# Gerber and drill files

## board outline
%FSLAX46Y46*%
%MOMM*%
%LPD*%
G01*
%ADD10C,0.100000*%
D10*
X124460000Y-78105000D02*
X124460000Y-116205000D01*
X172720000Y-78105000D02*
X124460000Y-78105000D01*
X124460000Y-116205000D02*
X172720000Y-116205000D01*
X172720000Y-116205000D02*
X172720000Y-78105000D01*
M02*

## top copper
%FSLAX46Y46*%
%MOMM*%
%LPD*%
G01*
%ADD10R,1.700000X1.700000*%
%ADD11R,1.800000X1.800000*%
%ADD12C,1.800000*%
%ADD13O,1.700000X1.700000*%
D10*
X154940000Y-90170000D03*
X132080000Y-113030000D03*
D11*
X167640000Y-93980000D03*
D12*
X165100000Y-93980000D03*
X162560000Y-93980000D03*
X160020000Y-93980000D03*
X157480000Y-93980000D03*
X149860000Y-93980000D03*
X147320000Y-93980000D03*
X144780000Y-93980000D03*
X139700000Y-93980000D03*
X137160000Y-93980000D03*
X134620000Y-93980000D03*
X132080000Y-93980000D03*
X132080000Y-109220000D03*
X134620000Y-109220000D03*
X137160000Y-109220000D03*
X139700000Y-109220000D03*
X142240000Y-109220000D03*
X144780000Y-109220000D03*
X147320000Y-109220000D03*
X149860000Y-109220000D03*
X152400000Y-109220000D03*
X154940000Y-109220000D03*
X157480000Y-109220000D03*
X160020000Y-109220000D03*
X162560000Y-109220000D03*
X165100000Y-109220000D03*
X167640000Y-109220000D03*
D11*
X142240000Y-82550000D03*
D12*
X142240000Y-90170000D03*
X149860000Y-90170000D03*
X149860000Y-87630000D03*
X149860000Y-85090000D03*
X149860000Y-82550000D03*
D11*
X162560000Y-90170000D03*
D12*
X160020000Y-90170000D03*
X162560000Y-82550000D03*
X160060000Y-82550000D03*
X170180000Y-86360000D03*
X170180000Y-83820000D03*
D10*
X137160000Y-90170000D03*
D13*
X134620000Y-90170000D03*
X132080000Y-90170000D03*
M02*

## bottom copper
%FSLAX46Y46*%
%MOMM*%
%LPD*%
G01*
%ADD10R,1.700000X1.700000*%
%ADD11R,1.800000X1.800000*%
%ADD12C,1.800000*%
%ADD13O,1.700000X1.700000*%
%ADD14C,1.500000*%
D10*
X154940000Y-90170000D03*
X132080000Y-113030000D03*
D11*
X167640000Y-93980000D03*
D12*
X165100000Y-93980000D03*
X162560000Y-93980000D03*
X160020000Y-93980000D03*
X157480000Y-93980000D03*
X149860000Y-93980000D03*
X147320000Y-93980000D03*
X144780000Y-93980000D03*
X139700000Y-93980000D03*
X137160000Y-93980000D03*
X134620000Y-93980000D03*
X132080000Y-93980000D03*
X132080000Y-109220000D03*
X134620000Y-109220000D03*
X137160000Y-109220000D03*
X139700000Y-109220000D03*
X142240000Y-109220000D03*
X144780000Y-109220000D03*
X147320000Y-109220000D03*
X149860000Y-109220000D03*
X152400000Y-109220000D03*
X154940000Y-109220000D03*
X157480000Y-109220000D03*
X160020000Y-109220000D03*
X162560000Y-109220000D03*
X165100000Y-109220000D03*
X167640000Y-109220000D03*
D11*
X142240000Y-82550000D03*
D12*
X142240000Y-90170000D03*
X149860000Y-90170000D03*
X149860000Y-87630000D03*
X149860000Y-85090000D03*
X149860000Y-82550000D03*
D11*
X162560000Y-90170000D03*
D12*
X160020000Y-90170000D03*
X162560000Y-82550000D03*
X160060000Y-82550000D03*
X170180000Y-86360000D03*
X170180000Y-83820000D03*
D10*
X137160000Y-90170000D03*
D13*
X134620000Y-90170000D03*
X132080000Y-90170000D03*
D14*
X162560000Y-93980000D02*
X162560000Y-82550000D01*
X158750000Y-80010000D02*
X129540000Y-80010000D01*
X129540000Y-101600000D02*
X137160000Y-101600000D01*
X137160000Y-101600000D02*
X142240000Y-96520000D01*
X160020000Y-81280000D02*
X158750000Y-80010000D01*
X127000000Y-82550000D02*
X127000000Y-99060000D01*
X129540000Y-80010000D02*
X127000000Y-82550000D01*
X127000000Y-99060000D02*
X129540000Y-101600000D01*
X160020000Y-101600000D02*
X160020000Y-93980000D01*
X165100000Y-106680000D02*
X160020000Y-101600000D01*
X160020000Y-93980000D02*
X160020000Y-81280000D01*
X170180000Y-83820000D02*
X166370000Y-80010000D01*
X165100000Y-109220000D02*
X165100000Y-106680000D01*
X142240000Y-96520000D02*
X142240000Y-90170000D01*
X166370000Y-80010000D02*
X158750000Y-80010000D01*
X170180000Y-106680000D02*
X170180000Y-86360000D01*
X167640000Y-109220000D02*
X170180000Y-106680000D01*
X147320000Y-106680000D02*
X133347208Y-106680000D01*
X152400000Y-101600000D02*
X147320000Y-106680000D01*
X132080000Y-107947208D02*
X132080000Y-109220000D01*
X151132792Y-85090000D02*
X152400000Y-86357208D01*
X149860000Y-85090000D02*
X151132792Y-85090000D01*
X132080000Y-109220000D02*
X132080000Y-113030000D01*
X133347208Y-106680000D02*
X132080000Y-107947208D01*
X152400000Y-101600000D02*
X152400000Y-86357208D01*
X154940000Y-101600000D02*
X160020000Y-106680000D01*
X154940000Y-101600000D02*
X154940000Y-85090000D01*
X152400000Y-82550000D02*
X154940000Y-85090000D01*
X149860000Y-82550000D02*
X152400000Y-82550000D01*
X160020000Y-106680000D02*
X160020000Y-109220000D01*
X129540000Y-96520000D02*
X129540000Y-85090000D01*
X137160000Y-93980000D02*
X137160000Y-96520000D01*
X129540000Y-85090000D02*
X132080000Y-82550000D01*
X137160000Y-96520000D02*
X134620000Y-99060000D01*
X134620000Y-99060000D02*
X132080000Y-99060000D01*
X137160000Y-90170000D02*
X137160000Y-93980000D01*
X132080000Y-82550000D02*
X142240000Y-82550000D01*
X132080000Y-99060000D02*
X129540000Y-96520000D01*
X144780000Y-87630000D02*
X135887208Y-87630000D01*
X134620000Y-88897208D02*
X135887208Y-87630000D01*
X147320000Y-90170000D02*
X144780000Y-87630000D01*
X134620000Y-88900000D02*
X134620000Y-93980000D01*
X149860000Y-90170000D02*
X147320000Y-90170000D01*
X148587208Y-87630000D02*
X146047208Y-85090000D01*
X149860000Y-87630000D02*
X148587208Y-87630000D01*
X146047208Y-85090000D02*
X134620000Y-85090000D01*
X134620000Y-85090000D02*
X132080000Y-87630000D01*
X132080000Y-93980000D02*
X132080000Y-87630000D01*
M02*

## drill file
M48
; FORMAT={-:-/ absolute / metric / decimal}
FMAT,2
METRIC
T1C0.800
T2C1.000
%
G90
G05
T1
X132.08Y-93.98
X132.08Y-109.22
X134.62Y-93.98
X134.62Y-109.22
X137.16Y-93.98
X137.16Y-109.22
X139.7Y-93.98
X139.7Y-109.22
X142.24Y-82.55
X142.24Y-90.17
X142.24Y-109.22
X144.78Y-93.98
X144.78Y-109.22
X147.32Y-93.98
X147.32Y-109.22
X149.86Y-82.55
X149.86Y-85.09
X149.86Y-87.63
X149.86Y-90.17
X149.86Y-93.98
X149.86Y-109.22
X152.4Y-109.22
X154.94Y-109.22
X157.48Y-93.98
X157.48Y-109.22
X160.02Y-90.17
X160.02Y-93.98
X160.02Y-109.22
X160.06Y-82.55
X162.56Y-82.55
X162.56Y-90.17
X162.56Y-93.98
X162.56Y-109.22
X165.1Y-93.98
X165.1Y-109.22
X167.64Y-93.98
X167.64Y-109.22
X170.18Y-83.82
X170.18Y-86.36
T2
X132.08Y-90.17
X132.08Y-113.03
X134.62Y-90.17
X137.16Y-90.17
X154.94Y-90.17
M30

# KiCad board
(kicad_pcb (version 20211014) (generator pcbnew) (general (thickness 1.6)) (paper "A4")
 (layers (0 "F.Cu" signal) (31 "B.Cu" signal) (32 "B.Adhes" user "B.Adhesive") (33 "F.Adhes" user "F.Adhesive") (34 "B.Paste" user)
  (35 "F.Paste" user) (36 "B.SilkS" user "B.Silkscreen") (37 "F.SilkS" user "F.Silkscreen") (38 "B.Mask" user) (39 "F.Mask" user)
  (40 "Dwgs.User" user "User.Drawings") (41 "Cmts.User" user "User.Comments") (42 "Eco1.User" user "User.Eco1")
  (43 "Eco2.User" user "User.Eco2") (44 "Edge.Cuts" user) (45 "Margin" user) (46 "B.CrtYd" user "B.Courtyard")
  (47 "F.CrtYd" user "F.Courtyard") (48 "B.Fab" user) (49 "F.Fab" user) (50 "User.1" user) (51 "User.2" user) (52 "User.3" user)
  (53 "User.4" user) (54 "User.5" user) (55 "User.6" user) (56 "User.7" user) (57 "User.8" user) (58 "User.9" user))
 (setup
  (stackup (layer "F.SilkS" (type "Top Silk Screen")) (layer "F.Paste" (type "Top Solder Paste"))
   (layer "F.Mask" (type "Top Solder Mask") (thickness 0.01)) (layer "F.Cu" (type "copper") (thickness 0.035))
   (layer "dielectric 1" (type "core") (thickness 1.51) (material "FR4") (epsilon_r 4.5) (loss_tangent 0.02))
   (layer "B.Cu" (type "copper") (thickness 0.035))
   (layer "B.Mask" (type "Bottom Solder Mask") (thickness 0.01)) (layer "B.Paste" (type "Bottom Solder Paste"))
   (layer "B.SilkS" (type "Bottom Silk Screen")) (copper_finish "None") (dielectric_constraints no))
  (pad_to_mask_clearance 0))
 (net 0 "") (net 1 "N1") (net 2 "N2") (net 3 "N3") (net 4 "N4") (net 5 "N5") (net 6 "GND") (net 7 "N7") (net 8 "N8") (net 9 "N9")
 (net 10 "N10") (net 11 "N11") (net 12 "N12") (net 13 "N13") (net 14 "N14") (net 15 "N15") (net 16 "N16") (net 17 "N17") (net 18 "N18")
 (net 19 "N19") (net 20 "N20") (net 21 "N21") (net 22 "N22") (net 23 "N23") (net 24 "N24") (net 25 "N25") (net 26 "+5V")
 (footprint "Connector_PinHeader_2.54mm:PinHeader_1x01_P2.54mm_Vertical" (layer "F.Cu") (at 154.94 90.17)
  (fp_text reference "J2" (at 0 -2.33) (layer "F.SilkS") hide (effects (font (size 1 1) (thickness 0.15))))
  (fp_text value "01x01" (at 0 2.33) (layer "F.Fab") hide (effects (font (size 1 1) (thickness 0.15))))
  (pad "1" thru_hole rect (at 0 0) (size 1.7 1.7) (drill 1) (layers *.Cu *.Mask) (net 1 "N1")))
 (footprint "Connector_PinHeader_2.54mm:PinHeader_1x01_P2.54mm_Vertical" (layer "F.Cu") (at 132.08 113.03 -90)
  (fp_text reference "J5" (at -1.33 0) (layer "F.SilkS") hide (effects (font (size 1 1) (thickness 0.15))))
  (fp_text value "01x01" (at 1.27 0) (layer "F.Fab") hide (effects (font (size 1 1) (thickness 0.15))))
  (pad "1" thru_hole rect (at 0 0 270) (size 1.7 1.7) (drill 1) (layers *.Cu *.Mask) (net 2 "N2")))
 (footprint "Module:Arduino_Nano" (layer "F.Cu") (at 167.64 93.98 -90)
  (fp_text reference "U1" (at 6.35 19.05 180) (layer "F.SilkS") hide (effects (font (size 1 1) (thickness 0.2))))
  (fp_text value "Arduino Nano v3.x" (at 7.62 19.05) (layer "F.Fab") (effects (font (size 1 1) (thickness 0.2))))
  (pad "1" thru_hole rect (at 0 0 270) (size 1.8 1.8) (drill 0.8) (layers *.Cu *.Mask) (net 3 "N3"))
  (pad "2" thru_hole circle (at 0 2.54 270) (size 1.8 1.8) (drill 0.8) (layers *.Cu *.Mask) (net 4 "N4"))
  (pad "3" thru_hole circle (at 0 5.08 270) (size 1.8 1.8) (drill 0.8) (layers *.Cu *.Mask) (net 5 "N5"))
  (pad "4" thru_hole circle (at 0 7.62 270) (size 1.8 1.8) (drill 0.8) (layers *.Cu *.Mask) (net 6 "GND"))
  (pad "5" thru_hole circle (at 0 10.16 270) (size 1.8 1.8) (drill 0.8) (layers *.Cu *.Mask) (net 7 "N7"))
  (pad "8" thru_hole circle (at 0 17.78 270) (size 1.8 1.8) (drill 0.8) (layers *.Cu *.Mask) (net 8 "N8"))
  (pad "9" thru_hole circle (at 0 20.32 270) (size 1.8 1.8) (drill 0.8) (layers *.Cu *.Mask) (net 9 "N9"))
  (pad "10" thru_hole circle (at 0 22.86 270) (size 1.8 1.8) (drill 0.8) (layers *.Cu *.Mask) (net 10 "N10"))
  (pad "12" thru_hole circle (at 0 27.94 270) (size 1.8 1.8) (drill 0.8) (layers *.Cu *.Mask) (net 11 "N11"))
  (pad "13" thru_hole circle (at 0 30.48 270) (size 1.8 1.8) (drill 0.8) (layers *.Cu *.Mask) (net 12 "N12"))
  (pad "14" thru_hole circle (at 0 33.02 270) (size 1.8 1.8) (drill 0.8) (layers *.Cu *.Mask) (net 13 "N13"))
  (pad "15" thru_hole circle (at 0 35.56 270) (size 1.8 1.8) (drill 0.8) (layers *.Cu *.Mask) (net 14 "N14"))
  (pad "16" thru_hole circle (at 15.24 35.56 270) (size 1.8 1.8) (drill 0.8) (layers *.Cu *.Mask) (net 2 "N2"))
  (pad "17" thru_hole circle (at 15.24 33.02 270) (size 1.8 1.8) (drill 0.8) (layers *.Cu *.Mask) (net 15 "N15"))
  (pad "18" thru_hole circle (at 15.24 30.48 270) (size 1.8 1.8) (drill 0.8) (layers *.Cu *.Mask) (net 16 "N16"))
  (pad "19" thru_hole circle (at 15.24 27.94 270) (size 1.8 1.8) (drill 0.8) (layers *.Cu *.Mask) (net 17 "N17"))
  (pad "20" thru_hole circle (at 15.24 25.4 270) (size 1.8 1.8) (drill 0.8) (layers *.Cu *.Mask) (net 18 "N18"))
  (pad "21" thru_hole circle (at 15.24 22.86 270) (size 1.8 1.8) (drill 0.8) (layers *.Cu *.Mask) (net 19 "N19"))
  (pad "22" thru_hole circle (at 15.24 20.32 270) (size 1.8 1.8) (drill 0.8) (layers *.Cu *.Mask) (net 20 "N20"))
  (pad "23" thru_hole circle (at 15.24 17.78 270) (size 1.8 1.8) (drill 0.8) (layers *.Cu *.Mask) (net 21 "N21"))
  (pad "24" thru_hole circle (at 15.24 15.24 270) (size 1.8 1.8) (drill 0.8) (layers *.Cu *.Mask) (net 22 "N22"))
  (pad "25" thru_hole circle (at 15.24 12.7 270) (size 1.8 1.8) (drill 0.8) (layers *.Cu *.Mask) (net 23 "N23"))
  (pad "26" thru_hole circle (at 15.24 10.16 270) (size 1.8 1.8) (drill 0.8) (layers *.Cu *.Mask) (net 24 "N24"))
  (pad "27" thru_hole circle (at 15.24 7.62 270) (size 1.8 1.8) (drill 0.8) (layers *.Cu *.Mask) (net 1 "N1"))
  (pad "28" thru_hole circle (at 15.24 5.08 270) (size 1.8 1.8) (drill 0.8) (layers *.Cu *.Mask) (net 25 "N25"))
  (pad "29" thru_hole circle (at 15.24 2.54 270) (size 1.8 1.8) (drill 0.8) (layers *.Cu *.Mask) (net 6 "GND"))
  (pad "30" thru_hole circle (at 15.24 0 270) (size 1.8 1.8) (drill 0.8) (layers *.Cu *.Mask) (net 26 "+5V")))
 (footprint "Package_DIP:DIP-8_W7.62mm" (layer "F.Cu") (at 142.24 82.55)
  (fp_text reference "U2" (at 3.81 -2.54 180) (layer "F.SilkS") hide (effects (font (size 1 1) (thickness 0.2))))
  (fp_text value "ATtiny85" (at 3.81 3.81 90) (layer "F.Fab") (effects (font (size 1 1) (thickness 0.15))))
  (pad "1" thru_hole rect (at 0 0) (size 1.8 1.8) (drill 0.8) (layers *.Cu *.Mask) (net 12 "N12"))
  (pad "4" thru_hole circle (at 0 7.62) (size 1.8 1.8) (drill 0.8) (layers *.Cu *.Mask) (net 6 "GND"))
  (pad "5" thru_hole circle (at 7.62 7.62) (size 1.8 1.8) (drill 0.8) (layers *.Cu *.Mask) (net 13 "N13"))
  (pad "6" thru_hole circle (at 7.62 5.08) (size 1.8 1.8) (drill 0.8) (layers *.Cu *.Mask) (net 14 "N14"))
  (pad "7" thru_hole circle (at 7.62 2.54) (size 1.8 1.8) (drill 0.8) (layers *.Cu *.Mask) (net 2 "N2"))
  (pad "8" thru_hole circle (at 7.62 0) (size 1.8 1.8) (drill 0.8) (layers *.Cu *.Mask) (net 1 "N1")))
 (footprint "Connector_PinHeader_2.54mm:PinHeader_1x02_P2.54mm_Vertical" (layer "F.Cu") (at 162.56 90.17 -90)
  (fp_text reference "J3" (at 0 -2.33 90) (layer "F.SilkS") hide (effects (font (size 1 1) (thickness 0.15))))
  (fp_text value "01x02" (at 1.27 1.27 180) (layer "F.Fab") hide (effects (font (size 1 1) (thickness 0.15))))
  (pad "1" thru_hole rect (at 0 0 270) (size 1.8 1.8) (drill 0.8) (layers *.Cu *.Mask) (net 5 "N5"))
  (pad "2" thru_hole circle (at 0 2.54 270) (size 1.8 1.8) (drill 0.8) (layers *.Cu *.Mask) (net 6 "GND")))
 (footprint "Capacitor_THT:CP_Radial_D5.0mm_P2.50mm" (layer "F.Cu") (at 162.56 82.55 180)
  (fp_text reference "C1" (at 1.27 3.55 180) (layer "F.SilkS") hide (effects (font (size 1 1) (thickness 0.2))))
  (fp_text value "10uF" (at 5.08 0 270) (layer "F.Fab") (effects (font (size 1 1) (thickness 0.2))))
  (pad "1" thru_hole circle (at 0 0 180) (size 1.8 1.8) (drill 0.8) (layers *.Cu *.Mask) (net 5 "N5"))
  (pad "2" thru_hole circle (at 2.5 0 180) (size 1.8 1.8) (drill 0.8) (layers *.Cu *.Mask) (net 6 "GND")))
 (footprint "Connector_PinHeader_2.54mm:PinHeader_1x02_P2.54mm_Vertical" (layer "F.Cu") (at 170.18 86.36 180)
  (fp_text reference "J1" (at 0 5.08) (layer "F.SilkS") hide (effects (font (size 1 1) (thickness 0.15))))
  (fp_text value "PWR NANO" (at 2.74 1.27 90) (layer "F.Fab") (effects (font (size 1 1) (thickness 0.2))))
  (pad "1" thru_hole circle (at 0 0 180) (size 1.8 1.8) (drill 0.8) (layers *.Cu *.Mask) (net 26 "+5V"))
  (pad "2" thru_hole circle (at 0 2.54 180) (size 1.8 1.8) (drill 0.8) (layers *.Cu *.Mask) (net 6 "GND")))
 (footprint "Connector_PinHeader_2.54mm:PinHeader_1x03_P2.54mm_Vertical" (layer "F.Cu") (at 137.16 90.17 -90)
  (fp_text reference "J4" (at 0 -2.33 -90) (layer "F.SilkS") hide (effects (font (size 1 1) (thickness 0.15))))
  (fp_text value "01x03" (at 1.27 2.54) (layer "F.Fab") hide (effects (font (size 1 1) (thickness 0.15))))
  (pad "1" thru_hole rect (at 0 0 270) (size 1.7 1.7) (drill 1) (layers *.Cu *.Mask) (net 12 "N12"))
  (pad "2" thru_hole oval (at 0 2.54 270) (size 1.7 1.7) (drill 1) (layers *.Cu *.Mask) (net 13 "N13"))
  (pad "3" thru_hole oval (at 0 5.08 270) (size 1.7 1.7) (drill 1) (layers *.Cu *.Mask) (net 14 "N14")))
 (gr_line (start 124.46 78.105) (end 124.46 116.205) (layer "Edge.Cuts") (width 0.1))
 (gr_line (start 172.72 78.105) (end 124.46 78.105) (layer "Edge.Cuts") (width 0.1))
 (gr_line (start 124.46 116.205) (end 172.72 116.205) (layer "Edge.Cuts") (width 0.1))
 (gr_line (start 172.72 116.205) (end 172.72 78.105) (layer "Edge.Cuts") (width 0.1))
 (segment (start 162.56 93.98) (end 162.56 82.55) (width 1.5) (layer "B.Cu") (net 5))
 (segment (start 158.75 80.01) (end 129.54 80.01) (width 1.5) (layer "B.Cu") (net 6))
 (segment (start 129.54 101.6) (end 137.16 101.6) (width 1.5) (layer "B.Cu") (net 6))
 (segment (start 137.16 101.6) (end 142.24 96.52) (width 1.5) (layer "B.Cu") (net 6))
 (segment (start 160.02 81.28) (end 158.75 80.01) (width 1.5) (layer "B.Cu") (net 6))
 (segment (start 127 82.55) (end 127 99.06) (width 1.5) (layer "B.Cu") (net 6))
 (segment (start 129.54 80.01) (end 127 82.55) (width 1.5) (layer "B.Cu") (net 6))
 (segment (start 127 99.06) (end 129.54 101.6) (width 1.5) (layer "B.Cu") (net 6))
 (segment (start 160.02 101.6) (end 160.02 93.98) (width 1.5) (layer "B.Cu") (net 6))
 (segment (start 165.1 106.68) (end 160.02 101.6) (width 1.5) (layer "B.Cu") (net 6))
 (segment (start 160.02 93.98) (end 160.02 81.28) (width 1.5) (layer "B.Cu") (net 6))
 (segment (start 170.18 83.82) (end 166.37 80.01) (width 1.5) (layer "B.Cu") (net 6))
 (segment (start 165.1 109.22) (end 165.1 106.68) (width 1.5) (layer "B.Cu") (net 6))
 (segment (start 142.24 96.52) (end 142.24 90.17) (width 1.5) (layer "B.Cu") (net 6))
 (segment (start 166.37 80.01) (end 158.75 80.01) (width 1.5) (layer "B.Cu") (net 6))
 (segment (start 170.18 106.68) (end 170.18 86.36) (width 1.5) (layer "B.Cu") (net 26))
 (segment (start 167.64 109.22) (end 170.18 106.68) (width 1.5) (layer "B.Cu") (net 26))
 (segment (start 147.32 106.68) (end 133.347208 106.68) (width 1.5) (layer "B.Cu") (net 2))
 (segment (start 152.4 101.6) (end 147.32 106.68) (width 1.5) (layer "B.Cu") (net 2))
 (segment (start 132.08 107.947208) (end 132.08 109.22) (width 1.5) (layer "B.Cu") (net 2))
 (segment (start 151.132792 85.09) (end 152.4 86.357208) (width 1.5) (layer "B.Cu") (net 2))
 (segment (start 149.86 85.09) (end 151.132792 85.09) (width 1.5) (layer "B.Cu") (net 2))
 (segment (start 132.08 109.22) (end 132.08 113.03) (width 1.5) (layer "B.Cu") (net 2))
 (segment (start 133.347208 106.68) (end 132.08 107.947208) (width 1.5) (layer "B.Cu") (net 2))
 (segment (start 152.4 101.6) (end 152.4 86.357208) (width 1.5) (layer "B.Cu") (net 2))
 (segment (start 154.94 101.6) (end 160.02 106.68) (width 1.5) (layer "B.Cu") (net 1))
 (segment (start 154.94 101.6) (end 154.94 85.09) (width 1.5) (layer "B.Cu") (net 1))
 (segment (start 152.4 82.55) (end 154.94 85.09) (width 1.5) (layer "B.Cu") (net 1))
 (segment (start 149.86 82.55) (end 152.4 82.55) (width 1.5) (layer "B.Cu") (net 1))
 (segment (start 160.02 106.68) (end 160.02 109.22) (width 1.5) (layer "B.Cu") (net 1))
 (segment (start 129.54 96.52) (end 129.54 85.09) (width 1.5) (layer "B.Cu") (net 12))
 (segment (start 137.16 93.98) (end 137.16 96.52) (width 1.5) (layer "B.Cu") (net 12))
 (segment (start 129.54 85.09) (end 132.08 82.55) (width 1.5) (layer "B.Cu") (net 12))
 (segment (start 137.16 96.52) (end 134.62 99.06) (width 1.5) (layer "B.Cu") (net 12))
 (segment (start 134.62 99.06) (end 132.08 99.06) (width 1.5) (layer "B.Cu") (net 12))
 (segment (start 137.16 90.17) (end 137.16 93.98) (width 1.5) (layer "B.Cu") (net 12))
 (segment (start 132.08 82.55) (end 142.24 82.55) (width 1.5) (layer "B.Cu") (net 12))
 (segment (start 132.08 99.06) (end 129.54 96.52) (width 1.5) (layer "B.Cu") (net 12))
 (segment (start 144.78 87.63) (end 135.887208 87.63) (width 1.5) (layer "B.Cu") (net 13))
 (segment (start 134.62 88.897208) (end 135.887208 87.63) (width 1.5) (layer "B.Cu") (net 13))
 (segment (start 147.32 90.17) (end 144.78 87.63) (width 1.5) (layer "B.Cu") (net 13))
 (segment (start 134.62 88.9) (end 134.62 93.98) (width 1.5) (layer "B.Cu") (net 13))
 (segment (start 149.86 90.17) (end 147.32 90.17) (width 1.5) (layer "B.Cu") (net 13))
 (segment (start 148.587208 87.63) (end 146.047208 85.09) (width 1.5) (layer "B.Cu") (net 14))
 (segment (start 149.86 87.63) (end 148.587208 87.63) (width 1.5) (layer "B.Cu") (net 14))
 (segment (start 146.047208 85.09) (end 134.62 85.09) (width 1.5) (layer "B.Cu") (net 14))
 (segment (start 134.62 85.09) (end 132.08 87.63) (width 1.5) (layer "B.Cu") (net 14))
 (segment (start 132.08 93.98) (end 132.08 87.63) (width 1.5) (layer "B.Cu") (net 14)))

